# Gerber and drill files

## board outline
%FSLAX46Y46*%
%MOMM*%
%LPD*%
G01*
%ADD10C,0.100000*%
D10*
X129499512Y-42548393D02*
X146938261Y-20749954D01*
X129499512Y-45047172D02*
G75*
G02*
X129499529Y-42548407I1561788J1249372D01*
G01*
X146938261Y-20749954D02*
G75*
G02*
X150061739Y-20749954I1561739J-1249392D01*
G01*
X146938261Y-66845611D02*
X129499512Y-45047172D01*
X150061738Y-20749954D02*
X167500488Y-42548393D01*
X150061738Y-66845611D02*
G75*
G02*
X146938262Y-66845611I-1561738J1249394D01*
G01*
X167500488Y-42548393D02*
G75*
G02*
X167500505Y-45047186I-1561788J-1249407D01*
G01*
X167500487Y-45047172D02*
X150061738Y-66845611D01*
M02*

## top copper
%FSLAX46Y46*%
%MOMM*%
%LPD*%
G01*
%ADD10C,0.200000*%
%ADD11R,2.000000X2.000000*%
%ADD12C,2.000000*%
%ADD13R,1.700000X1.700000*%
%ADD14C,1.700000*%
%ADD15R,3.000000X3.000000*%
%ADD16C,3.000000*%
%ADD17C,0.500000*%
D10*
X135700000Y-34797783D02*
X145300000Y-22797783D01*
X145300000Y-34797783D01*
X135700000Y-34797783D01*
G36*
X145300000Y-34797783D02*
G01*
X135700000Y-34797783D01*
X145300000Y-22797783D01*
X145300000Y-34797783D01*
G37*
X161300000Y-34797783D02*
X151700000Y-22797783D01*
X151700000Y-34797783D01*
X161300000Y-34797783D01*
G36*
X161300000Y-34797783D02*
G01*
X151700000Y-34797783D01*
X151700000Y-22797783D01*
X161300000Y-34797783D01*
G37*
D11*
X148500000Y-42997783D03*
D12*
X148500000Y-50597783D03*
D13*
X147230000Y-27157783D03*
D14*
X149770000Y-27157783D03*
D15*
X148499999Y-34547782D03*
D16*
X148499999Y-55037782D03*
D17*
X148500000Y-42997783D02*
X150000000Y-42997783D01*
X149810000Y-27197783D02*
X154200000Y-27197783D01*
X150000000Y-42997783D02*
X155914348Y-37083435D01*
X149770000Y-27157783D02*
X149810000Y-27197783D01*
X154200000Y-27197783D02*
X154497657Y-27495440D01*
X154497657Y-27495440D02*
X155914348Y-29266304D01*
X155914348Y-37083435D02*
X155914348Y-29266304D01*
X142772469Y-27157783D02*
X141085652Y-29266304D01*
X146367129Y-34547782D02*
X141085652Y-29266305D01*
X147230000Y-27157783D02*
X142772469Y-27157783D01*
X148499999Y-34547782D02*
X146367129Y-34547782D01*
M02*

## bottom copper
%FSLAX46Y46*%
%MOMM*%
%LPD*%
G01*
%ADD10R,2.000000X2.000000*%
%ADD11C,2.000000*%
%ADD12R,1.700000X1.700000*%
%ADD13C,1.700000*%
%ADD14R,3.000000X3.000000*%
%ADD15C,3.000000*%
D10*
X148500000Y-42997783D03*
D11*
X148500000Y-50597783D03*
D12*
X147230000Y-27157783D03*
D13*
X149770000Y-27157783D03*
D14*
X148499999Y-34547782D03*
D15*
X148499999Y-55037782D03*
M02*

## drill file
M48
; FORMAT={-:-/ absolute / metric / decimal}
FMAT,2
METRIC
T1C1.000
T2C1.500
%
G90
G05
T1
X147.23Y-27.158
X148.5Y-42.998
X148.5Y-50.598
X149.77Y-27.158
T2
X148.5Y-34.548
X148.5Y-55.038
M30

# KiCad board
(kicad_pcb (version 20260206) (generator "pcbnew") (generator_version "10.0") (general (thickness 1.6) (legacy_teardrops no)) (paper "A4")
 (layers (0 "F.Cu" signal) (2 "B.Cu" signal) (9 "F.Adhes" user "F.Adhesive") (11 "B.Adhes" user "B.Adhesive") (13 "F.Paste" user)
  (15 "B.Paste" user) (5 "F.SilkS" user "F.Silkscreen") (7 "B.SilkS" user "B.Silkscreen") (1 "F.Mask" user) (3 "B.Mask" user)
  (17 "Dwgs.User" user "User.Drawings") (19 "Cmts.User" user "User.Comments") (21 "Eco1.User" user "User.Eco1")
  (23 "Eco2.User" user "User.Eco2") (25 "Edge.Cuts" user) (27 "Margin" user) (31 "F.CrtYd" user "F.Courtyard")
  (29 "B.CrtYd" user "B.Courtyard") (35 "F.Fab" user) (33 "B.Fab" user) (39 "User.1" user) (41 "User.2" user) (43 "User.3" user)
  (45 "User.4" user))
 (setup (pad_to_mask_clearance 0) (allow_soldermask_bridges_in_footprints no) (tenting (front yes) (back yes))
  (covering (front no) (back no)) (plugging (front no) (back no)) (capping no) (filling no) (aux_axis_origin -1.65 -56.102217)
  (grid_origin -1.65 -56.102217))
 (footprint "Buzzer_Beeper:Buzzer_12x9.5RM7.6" (layer "F.Cu") (at 148.5 42.997783 -90)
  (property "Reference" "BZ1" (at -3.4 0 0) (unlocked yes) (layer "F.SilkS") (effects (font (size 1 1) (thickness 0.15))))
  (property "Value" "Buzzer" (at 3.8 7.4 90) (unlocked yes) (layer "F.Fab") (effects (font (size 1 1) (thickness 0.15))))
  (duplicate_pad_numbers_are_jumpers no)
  (pad "1" thru_hole rect (at 0 0 270) (size 2 2) (drill 1) (layers "*.Cu" "*.Mask") (remove_unused_layers no) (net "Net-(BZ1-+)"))
  (pad "2" thru_hole circle (at 7.6 0 270) (size 2 2) (drill 1) (layers "*.Cu" "*.Mask") (remove_unused_layers no) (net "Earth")))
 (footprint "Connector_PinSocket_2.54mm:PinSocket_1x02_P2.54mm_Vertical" (layer "F.Cu") (at 147.23 27.157783 90)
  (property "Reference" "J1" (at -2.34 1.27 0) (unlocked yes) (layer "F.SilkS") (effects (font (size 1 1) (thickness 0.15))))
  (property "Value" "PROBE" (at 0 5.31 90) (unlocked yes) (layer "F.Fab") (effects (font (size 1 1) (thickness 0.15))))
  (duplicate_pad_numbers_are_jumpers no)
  (pad "1" thru_hole rect (at 0 0 90) (size 1.7 1.7) (drill 1) (layers "*.Cu" "*.Mask") (remove_unused_layers no) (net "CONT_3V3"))
  (pad "2" thru_hole circle (at 0 2.54 90) (size 1.7 1.7) (drill 1) (layers "*.Cu" "*.Mask") (remove_unused_layers no) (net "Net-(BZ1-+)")))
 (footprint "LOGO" (layer "B.Cu") (at 159.439472 39.132096 -45)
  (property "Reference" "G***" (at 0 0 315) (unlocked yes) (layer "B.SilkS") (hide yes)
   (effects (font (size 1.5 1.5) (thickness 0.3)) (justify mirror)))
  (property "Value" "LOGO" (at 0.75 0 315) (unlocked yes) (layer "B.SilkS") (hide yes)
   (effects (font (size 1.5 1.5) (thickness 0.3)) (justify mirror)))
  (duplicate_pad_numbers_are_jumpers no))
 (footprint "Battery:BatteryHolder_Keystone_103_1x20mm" (layer "B.Cu") (at 148.499999 34.547782 -90)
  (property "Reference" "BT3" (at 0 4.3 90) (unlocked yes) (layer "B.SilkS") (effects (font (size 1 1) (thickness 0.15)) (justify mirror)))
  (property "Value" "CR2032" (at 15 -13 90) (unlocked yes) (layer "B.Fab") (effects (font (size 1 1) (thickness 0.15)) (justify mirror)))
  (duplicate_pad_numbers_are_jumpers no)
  (pad "1" thru_hole rect (at 0 0 270) (size 3 3) (drill 1.5) (layers "*.Cu" "*.Mask") (remove_unused_layers no) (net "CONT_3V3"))
  (pad "2" thru_hole circle (at 20.49 0 270) (size 3 3) (drill 1.5) (layers "*.Cu" "*.Mask") (remove_unused_layers no) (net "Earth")))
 (gr_poly
  (pts (xy 135.7 34.797783) (xy 145.3 22.797783) (xy 145.3 34.797783)) (stroke (width 0.2) (type solid)) (fill yes) (layers "F.Cu" "F.Mask")
  (net "CONT_3V3"))
 (gr_poly
  (pts (xy 161.3 34.797783) (xy 151.7 22.797783) (xy 151.7 34.797783)) (stroke (width 0.2) (type solid)) (fill yes) (layers "F.Cu" "F.Mask")
  (net "Net-(BZ1-+)"))
 (gr_line (start 129.499512 42.548393) (end 146.938261 20.749954) (stroke (width 0.1) (type default)) (layer "Edge.Cuts"))
 (gr_arc (start 129.499512 45.047172) (mid 129.06126 43.797783) (end 129.499512 42.548393) (stroke (width 0.1) (type default))
  (layer "Edge.Cuts"))
 (gr_arc (start 146.938261 20.749954) (mid 148.5 19.999344) (end 150.061738 20.749954) (stroke (width 0.1) (type default))
  (layer "Edge.Cuts"))
 (gr_line (start 146.938261 66.845611) (end 129.499512 45.047172) (stroke (width 0.1) (type default)) (layer "Edge.Cuts"))
 (gr_line (start 150.061738 20.749954) (end 167.500488 42.548393) (stroke (width 0.1) (type default)) (layer "Edge.Cuts"))
 (gr_arc (start 150.061738 66.845611) (mid 148.5 67.59622) (end 146.938261 66.845611) (stroke (width 0.1) (type default))
  (layer "Edge.Cuts"))
 (gr_arc (start 167.500488 42.548393) (mid 167.938739 43.797782) (end 167.500487 45.047172) (stroke (width 0.1) (type default))
  (layer "Edge.Cuts"))
 (gr_line (start 167.500487 45.047172) (end 150.061738 66.845611) (stroke (width 0.1) (type default)) (layer "Edge.Cuts"))
 (segment (start 148.5 42.997783) (end 150 42.997783) (width 0.5) (layer "F.Cu") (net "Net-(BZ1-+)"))
 (segment (start 149.81 27.197783) (end 154.2 27.197783) (width 0.5) (layer "F.Cu") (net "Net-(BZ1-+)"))
 (segment (start 150 42.997783) (end 155.914348 37.083435) (width 0.5) (layer "F.Cu") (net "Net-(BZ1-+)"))
 (segment (start 149.77 27.157783) (end 149.81 27.197783) (width 0.5) (layer "F.Cu") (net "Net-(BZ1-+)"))
 (segment (start 154.2 27.197783) (end 154.497657 27.49544) (width 0.5) (layer "F.Cu") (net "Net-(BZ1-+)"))
 (segment (start 154.497657 27.49544) (end 155.914348 29.266304) (width 0.5) (layer "F.Cu") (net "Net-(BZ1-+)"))
 (segment (start 155.914348 37.083435) (end 155.914348 29.266304) (width 0.5) (layer "F.Cu") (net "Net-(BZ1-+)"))
 (segment (start 142.772469 27.157783) (end 141.085652 29.266304) (width 0.5) (layer "F.Cu") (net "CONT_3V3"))
 (segment (start 146.367129 34.547782) (end 141.085652 29.266305) (width 0.5) (layer "F.Cu") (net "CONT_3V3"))
 (segment (start 147.23 27.157783) (end 142.772469 27.157783) (width 0.5) (layer "F.Cu") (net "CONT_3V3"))
 (segment (start 148.499999 34.547782) (end 146.367129 34.547782) (width 0.5) (layer "F.Cu") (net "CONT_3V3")))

